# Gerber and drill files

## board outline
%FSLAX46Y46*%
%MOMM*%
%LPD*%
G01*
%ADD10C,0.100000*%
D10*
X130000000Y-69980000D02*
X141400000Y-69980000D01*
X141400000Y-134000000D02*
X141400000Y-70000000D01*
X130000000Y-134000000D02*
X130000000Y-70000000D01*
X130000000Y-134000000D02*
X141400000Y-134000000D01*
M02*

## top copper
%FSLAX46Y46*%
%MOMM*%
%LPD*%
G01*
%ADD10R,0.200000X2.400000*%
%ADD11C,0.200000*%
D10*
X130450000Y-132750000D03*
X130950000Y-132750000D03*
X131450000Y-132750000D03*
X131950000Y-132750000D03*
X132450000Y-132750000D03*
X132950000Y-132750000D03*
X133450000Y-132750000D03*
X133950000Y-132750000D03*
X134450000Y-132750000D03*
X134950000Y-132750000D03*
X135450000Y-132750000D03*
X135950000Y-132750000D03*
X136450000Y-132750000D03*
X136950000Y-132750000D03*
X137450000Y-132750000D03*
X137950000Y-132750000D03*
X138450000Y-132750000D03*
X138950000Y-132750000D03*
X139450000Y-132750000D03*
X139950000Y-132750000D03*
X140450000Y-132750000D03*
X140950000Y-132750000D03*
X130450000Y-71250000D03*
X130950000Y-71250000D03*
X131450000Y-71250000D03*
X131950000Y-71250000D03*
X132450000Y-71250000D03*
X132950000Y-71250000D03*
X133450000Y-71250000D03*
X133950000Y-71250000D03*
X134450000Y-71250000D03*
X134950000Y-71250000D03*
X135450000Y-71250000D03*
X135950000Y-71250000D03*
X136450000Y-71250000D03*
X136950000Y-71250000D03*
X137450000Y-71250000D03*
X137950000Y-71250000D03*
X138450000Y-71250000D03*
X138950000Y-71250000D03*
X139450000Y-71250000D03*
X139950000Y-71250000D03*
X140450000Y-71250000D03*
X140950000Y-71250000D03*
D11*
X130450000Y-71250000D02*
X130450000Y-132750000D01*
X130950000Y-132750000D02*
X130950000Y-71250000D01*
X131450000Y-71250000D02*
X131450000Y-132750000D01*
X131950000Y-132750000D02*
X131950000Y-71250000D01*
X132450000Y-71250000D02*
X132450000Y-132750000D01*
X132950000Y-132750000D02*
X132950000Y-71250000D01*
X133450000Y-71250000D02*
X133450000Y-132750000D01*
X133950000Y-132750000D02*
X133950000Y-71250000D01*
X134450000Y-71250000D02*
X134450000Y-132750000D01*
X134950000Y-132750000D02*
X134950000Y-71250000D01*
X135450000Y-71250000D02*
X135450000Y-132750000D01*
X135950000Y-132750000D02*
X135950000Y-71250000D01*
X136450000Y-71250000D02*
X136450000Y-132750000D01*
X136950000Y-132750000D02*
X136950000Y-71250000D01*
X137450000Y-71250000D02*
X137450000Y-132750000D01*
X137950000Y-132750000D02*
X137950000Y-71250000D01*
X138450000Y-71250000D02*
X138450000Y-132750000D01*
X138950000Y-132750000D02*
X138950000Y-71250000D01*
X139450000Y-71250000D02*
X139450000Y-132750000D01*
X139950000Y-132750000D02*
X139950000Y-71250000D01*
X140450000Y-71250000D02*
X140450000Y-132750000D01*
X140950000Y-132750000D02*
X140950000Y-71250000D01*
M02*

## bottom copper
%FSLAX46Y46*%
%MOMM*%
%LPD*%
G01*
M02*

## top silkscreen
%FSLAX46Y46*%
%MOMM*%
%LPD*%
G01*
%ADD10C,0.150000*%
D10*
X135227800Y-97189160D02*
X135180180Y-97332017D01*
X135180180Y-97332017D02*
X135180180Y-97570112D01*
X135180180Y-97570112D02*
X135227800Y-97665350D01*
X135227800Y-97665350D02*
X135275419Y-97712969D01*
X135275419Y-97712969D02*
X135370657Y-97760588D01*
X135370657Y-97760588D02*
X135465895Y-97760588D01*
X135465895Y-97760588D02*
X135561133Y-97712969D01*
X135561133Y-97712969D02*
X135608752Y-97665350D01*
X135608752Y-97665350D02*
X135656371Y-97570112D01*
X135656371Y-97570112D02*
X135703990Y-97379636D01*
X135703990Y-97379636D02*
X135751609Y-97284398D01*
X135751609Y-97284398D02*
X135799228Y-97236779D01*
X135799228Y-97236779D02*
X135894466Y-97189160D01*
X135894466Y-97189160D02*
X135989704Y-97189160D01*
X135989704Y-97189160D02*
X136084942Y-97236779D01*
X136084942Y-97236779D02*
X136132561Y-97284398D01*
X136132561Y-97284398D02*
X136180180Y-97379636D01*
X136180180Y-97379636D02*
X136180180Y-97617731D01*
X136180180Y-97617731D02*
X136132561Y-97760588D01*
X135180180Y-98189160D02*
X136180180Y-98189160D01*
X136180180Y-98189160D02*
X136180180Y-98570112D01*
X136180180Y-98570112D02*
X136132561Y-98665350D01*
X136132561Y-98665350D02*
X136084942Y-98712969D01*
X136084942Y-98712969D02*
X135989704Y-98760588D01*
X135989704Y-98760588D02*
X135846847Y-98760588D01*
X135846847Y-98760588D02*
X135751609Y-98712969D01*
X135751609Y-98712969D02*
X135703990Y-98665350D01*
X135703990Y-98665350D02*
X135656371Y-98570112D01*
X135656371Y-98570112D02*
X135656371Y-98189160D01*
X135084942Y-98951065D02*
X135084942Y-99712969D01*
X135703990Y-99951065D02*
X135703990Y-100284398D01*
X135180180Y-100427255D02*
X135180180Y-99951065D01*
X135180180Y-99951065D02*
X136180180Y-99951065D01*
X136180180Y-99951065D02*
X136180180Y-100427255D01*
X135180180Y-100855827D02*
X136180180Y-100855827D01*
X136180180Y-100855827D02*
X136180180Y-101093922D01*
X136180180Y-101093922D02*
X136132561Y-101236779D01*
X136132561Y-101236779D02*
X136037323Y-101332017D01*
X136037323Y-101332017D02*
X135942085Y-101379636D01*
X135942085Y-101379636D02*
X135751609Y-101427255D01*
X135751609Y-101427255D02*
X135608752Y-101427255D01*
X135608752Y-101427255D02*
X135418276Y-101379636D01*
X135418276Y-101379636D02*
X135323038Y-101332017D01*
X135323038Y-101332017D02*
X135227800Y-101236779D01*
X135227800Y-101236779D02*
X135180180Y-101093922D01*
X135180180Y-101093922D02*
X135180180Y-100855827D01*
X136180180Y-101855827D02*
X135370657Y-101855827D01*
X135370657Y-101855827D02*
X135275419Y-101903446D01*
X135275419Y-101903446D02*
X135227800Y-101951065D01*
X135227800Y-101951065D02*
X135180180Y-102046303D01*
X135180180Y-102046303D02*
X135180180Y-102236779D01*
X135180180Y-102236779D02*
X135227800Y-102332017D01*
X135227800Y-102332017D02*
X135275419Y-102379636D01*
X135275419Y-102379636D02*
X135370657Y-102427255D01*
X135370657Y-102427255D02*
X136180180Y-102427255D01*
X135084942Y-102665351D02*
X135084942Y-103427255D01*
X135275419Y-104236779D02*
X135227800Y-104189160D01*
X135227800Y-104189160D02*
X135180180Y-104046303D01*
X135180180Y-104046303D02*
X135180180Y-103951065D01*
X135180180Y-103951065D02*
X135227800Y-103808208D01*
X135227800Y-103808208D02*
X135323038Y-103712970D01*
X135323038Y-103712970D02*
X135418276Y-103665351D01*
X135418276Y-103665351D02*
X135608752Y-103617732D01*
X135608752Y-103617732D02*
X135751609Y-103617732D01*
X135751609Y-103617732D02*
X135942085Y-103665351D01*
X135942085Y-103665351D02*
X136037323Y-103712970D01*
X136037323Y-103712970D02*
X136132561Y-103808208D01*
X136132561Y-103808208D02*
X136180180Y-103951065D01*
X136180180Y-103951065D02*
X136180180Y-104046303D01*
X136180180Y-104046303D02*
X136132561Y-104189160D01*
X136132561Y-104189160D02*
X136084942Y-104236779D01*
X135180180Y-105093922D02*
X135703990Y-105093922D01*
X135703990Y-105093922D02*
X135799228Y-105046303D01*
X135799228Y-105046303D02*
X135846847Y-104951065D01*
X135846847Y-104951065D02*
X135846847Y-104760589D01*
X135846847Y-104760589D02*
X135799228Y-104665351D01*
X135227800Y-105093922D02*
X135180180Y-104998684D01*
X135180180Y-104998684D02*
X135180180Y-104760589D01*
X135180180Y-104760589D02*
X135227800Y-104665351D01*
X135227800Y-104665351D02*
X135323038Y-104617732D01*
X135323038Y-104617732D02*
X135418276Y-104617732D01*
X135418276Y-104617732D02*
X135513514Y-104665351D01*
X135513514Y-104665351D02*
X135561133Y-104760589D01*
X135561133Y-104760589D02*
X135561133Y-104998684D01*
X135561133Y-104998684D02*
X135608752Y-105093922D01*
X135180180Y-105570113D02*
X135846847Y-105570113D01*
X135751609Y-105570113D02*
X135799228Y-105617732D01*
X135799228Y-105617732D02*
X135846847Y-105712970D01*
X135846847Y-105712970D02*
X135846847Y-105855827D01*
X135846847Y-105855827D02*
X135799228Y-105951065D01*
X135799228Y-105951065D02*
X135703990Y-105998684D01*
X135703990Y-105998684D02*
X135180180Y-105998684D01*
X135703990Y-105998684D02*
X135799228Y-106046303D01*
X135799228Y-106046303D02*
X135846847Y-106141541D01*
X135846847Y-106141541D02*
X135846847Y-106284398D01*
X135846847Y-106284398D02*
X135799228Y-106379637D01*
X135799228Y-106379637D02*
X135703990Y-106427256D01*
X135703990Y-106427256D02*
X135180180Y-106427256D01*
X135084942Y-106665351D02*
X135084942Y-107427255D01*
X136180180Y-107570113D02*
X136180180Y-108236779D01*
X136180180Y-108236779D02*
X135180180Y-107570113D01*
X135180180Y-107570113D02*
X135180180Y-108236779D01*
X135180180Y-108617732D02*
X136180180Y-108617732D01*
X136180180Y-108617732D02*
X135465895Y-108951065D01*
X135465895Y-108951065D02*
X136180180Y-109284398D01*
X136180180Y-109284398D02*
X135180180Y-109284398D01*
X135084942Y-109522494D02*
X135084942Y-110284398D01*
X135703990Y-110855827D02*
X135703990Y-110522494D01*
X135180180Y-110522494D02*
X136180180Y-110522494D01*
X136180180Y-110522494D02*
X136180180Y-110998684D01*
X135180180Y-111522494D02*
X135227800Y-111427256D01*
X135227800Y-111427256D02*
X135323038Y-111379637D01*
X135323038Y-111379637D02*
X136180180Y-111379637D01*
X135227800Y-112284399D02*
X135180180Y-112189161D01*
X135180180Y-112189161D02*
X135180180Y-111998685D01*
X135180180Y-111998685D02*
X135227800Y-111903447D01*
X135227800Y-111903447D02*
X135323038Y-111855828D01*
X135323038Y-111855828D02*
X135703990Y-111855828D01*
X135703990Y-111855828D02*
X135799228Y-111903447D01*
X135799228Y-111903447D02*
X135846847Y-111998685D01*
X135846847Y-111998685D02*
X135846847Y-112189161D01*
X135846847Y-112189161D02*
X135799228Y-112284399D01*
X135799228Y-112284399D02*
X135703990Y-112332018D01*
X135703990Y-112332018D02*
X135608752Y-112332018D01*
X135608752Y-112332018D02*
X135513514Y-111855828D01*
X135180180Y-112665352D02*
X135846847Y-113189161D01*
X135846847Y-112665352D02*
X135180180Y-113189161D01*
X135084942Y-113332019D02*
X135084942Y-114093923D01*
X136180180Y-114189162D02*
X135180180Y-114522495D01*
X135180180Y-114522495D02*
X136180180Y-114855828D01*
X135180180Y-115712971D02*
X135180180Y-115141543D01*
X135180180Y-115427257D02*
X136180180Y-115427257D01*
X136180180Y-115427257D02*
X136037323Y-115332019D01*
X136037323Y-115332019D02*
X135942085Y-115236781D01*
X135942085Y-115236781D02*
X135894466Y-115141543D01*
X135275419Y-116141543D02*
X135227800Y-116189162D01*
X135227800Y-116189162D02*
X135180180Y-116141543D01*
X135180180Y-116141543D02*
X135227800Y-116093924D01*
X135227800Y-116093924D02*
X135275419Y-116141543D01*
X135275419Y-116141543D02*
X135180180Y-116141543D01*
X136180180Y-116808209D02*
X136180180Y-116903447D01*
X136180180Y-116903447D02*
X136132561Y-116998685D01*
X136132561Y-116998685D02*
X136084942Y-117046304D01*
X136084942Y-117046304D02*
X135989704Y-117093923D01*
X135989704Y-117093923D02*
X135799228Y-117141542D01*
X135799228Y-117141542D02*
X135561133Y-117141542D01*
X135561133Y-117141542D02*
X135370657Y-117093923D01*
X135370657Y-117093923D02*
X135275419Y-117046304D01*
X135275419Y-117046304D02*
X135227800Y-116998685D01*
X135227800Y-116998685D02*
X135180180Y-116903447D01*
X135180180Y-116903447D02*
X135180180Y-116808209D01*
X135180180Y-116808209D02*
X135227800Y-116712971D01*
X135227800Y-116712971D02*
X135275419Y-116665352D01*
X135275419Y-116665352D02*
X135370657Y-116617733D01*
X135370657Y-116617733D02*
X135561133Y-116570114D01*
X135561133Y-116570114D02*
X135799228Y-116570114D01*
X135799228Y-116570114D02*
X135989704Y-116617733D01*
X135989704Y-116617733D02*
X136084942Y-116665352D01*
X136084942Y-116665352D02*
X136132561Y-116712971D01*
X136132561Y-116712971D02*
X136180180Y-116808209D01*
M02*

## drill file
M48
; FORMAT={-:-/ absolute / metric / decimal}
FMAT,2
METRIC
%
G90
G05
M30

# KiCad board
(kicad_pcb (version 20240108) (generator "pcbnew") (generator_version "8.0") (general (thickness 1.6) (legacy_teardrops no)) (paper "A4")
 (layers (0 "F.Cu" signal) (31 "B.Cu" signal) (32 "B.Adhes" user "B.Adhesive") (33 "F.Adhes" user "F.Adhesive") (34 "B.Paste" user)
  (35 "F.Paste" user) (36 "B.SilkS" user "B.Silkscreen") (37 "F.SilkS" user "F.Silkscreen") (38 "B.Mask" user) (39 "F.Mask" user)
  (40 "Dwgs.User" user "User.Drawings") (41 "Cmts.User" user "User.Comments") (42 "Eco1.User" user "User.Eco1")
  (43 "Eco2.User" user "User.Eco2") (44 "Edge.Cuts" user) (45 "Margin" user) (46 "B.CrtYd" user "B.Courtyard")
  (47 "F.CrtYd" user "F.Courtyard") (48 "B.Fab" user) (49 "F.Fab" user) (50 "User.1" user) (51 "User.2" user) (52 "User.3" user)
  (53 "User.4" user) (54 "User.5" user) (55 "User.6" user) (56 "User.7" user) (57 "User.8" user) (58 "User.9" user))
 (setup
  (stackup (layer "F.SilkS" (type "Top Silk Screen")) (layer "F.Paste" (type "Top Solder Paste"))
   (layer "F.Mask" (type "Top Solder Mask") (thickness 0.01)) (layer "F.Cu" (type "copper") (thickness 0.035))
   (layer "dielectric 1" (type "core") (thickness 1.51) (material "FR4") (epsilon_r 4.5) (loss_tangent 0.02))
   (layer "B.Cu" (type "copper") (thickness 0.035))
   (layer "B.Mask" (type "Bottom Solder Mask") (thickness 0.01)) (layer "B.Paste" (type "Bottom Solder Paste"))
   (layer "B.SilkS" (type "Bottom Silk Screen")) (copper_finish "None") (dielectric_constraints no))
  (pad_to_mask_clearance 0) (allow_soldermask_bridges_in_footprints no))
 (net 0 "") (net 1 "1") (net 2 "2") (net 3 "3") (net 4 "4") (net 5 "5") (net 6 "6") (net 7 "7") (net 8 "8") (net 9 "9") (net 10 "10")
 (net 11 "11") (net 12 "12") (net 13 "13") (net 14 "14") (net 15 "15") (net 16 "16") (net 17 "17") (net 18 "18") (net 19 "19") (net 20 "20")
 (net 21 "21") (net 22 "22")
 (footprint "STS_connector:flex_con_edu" (layer "F.Cu") (at 130 136.1)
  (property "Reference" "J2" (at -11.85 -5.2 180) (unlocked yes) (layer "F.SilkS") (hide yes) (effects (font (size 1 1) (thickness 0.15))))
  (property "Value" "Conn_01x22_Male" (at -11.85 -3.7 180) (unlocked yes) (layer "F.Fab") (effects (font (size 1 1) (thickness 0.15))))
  (pad "1" smd rect (at 0.45 -3.35) (size 0.2 2.4) (layers "F.Cu" "F.Paste" "F.Mask") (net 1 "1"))
  (pad "2" smd rect (at 0.95 -3.35) (size 0.2 2.4) (layers "F.Cu" "F.Paste" "F.Mask") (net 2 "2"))
  (pad "3" smd rect (at 1.45 -3.35) (size 0.2 2.4) (layers "F.Cu" "F.Paste" "F.Mask") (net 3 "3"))
  (pad "4" smd rect (at 1.95 -3.35) (size 0.2 2.4) (layers "F.Cu" "F.Paste" "F.Mask") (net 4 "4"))
  (pad "5" smd rect (at 2.45 -3.35) (size 0.2 2.4) (layers "F.Cu" "F.Paste" "F.Mask") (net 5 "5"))
  (pad "6" smd rect (at 2.95 -3.35) (size 0.2 2.4) (layers "F.Cu" "F.Paste" "F.Mask") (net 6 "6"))
  (pad "7" smd rect (at 3.45 -3.35) (size 0.2 2.4) (layers "F.Cu" "F.Paste" "F.Mask") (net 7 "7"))
  (pad "8" smd rect (at 3.95 -3.35) (size 0.2 2.4) (layers "F.Cu" "F.Paste" "F.Mask") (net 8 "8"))
  (pad "9" smd rect (at 4.45 -3.35) (size 0.2 2.4) (layers "F.Cu" "F.Paste" "F.Mask") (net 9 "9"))
  (pad "10" smd rect (at 4.95 -3.35) (size 0.2 2.4) (layers "F.Cu" "F.Paste" "F.Mask") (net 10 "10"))
  (pad "11" smd rect (at 5.45 -3.35) (size 0.2 2.4) (layers "F.Cu" "F.Paste" "F.Mask") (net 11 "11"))
  (pad "12" smd rect (at 5.95 -3.35) (size 0.2 2.4) (layers "F.Cu" "F.Paste" "F.Mask") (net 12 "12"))
  (pad "13" smd rect (at 6.45 -3.35) (size 0.2 2.4) (layers "F.Cu" "F.Paste" "F.Mask") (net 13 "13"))
  (pad "14" smd rect (at 6.95 -3.35) (size 0.2 2.4) (layers "F.Cu" "F.Paste" "F.Mask") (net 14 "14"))
  (pad "15" smd rect (at 7.45 -3.35) (size 0.2 2.4) (layers "F.Cu" "F.Paste" "F.Mask") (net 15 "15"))
  (pad "16" smd rect (at 7.95 -3.35) (size 0.2 2.4) (layers "F.Cu" "F.Paste" "F.Mask") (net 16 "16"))
  (pad "17" smd rect (at 8.45 -3.35) (size 0.2 2.4) (layers "F.Cu" "F.Paste" "F.Mask") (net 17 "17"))
  (pad "18" smd rect (at 8.95 -3.35) (size 0.2 2.4) (layers "F.Cu" "F.Paste" "F.Mask") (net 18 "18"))
  (pad "19" smd rect (at 9.45 -3.35) (size 0.2 2.4) (layers "F.Cu" "F.Paste" "F.Mask") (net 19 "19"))
  (pad "20" smd rect (at 9.95 -3.35) (size 0.2 2.4) (layers "F.Cu" "F.Paste" "F.Mask") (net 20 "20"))
  (pad "21" smd rect (at 10.45 -3.35) (size 0.2 2.4) (layers "F.Cu" "F.Paste" "F.Mask") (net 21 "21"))
  (pad "22" smd rect (at 10.95 -3.35) (size 0.2 2.4) (layers "F.Cu" "F.Paste" "F.Mask") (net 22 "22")))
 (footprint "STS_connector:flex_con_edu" (layer "F.Cu") (at 130 74.6)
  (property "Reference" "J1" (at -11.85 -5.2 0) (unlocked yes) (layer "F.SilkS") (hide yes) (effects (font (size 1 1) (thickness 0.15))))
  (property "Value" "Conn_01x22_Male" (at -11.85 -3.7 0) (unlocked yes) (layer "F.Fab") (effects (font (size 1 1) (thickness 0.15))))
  (pad "1" smd rect (at 0.45 -3.35) (size 0.2 2.4) (layers "F.Cu" "F.Paste" "F.Mask") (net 1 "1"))
  (pad "2" smd rect (at 0.95 -3.35) (size 0.2 2.4) (layers "F.Cu" "F.Paste" "F.Mask") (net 2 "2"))
  (pad "3" smd rect (at 1.45 -3.35) (size 0.2 2.4) (layers "F.Cu" "F.Paste" "F.Mask") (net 3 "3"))
  (pad "4" smd rect (at 1.95 -3.35) (size 0.2 2.4) (layers "F.Cu" "F.Paste" "F.Mask") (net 4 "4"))
  (pad "5" smd rect (at 2.45 -3.35) (size 0.2 2.4) (layers "F.Cu" "F.Paste" "F.Mask") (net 5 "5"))
  (pad "6" smd rect (at 2.95 -3.35) (size 0.2 2.4) (layers "F.Cu" "F.Paste" "F.Mask") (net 6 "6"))
  (pad "7" smd rect (at 3.45 -3.35) (size 0.2 2.4) (layers "F.Cu" "F.Paste" "F.Mask") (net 7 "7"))
  (pad "8" smd rect (at 3.95 -3.35) (size 0.2 2.4) (layers "F.Cu" "F.Paste" "F.Mask") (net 8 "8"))
  (pad "9" smd rect (at 4.45 -3.35) (size 0.2 2.4) (layers "F.Cu" "F.Paste" "F.Mask") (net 9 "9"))
  (pad "10" smd rect (at 4.95 -3.35) (size 0.2 2.4) (layers "F.Cu" "F.Paste" "F.Mask") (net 10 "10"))
  (pad "11" smd rect (at 5.45 -3.35) (size 0.2 2.4) (layers "F.Cu" "F.Paste" "F.Mask") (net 11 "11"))
  (pad "12" smd rect (at 5.95 -3.35) (size 0.2 2.4) (layers "F.Cu" "F.Paste" "F.Mask") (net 12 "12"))
  (pad "13" smd rect (at 6.45 -3.35) (size 0.2 2.4) (layers "F.Cu" "F.Paste" "F.Mask") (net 13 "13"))
  (pad "14" smd rect (at 6.95 -3.35) (size 0.2 2.4) (layers "F.Cu" "F.Paste" "F.Mask") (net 14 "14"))
  (pad "15" smd rect (at 7.45 -3.35) (size 0.2 2.4) (layers "F.Cu" "F.Paste" "F.Mask") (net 15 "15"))
  (pad "16" smd rect (at 7.95 -3.35) (size 0.2 2.4) (layers "F.Cu" "F.Paste" "F.Mask") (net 16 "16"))
  (pad "17" smd rect (at 8.45 -3.35) (size 0.2 2.4) (layers "F.Cu" "F.Paste" "F.Mask") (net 17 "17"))
  (pad "18" smd rect (at 8.95 -3.35) (size 0.2 2.4) (layers "F.Cu" "F.Paste" "F.Mask") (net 18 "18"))
  (pad "19" smd rect (at 9.45 -3.35) (size 0.2 2.4) (layers "F.Cu" "F.Paste" "F.Mask") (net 19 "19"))
  (pad "20" smd rect (at 9.95 -3.35) (size 0.2 2.4) (layers "F.Cu" "F.Paste" "F.Mask") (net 20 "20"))
  (pad "21" smd rect (at 10.45 -3.35) (size 0.2 2.4) (layers "F.Cu" "F.Paste" "F.Mask") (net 21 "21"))
  (pad "22" smd rect (at 10.95 -3.35) (size 0.2 2.4) (layers "F.Cu" "F.Paste" "F.Mask") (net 22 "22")))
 (gr_line (start 130 69.98) (end 141.4 69.98) (stroke (width 0.1) (type solid)) (layer "Edge.Cuts"))
 (gr_line (start 141.4 134) (end 141.4 70) (stroke (width 0.1) (type solid)) (layer "Edge.Cuts"))
 (gr_line (start 130 134) (end 130 70) (stroke (width 0.1) (type solid)) (layer "Edge.Cuts"))
 (gr_line (start 130 134) (end 141.4 134) (stroke (width 0.1) (type solid)) (layer "Edge.Cuts"))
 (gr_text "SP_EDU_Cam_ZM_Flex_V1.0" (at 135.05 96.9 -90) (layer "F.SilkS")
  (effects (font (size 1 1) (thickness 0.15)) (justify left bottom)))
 (segment (start 130.45 71.25) (end 130.45 132.75) (width 0.2) (layer "F.Cu") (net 1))
 (segment (start 130.95 132.75) (end 130.95 71.25) (width 0.2) (layer "F.Cu") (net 2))
 (segment (start 131.45 71.25) (end 131.45 132.75) (width 0.2) (layer "F.Cu") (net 3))
 (segment (start 131.95 132.75) (end 131.95 71.25) (width 0.2) (layer "F.Cu") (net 4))
 (segment (start 132.45 71.25) (end 132.45 132.75) (width 0.2) (layer "F.Cu") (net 5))
 (segment (start 132.95 132.75) (end 132.95 71.25) (width 0.2) (layer "F.Cu") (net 6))
 (segment (start 133.45 71.25) (end 133.45 132.75) (width 0.2) (layer "F.Cu") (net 7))
 (segment (start 133.95 132.75) (end 133.95 71.25) (width 0.2) (layer "F.Cu") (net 8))
 (segment (start 134.45 71.25) (end 134.45 132.75) (width 0.2) (layer "F.Cu") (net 9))
 (segment (start 134.95 132.75) (end 134.95 71.25) (width 0.2) (layer "F.Cu") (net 10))
 (segment (start 135.45 71.25) (end 135.45 132.75) (width 0.2) (layer "F.Cu") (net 11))
 (segment (start 135.95 132.75) (end 135.95 71.25) (width 0.2) (layer "F.Cu") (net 12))
 (segment (start 136.45 71.25) (end 136.45 132.75) (width 0.2) (layer "F.Cu") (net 13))
 (segment (start 136.95 132.75) (end 136.95 71.25) (width 0.2) (layer "F.Cu") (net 14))
 (segment (start 137.45 71.25) (end 137.45 132.75) (width 0.2) (layer "F.Cu") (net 15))
 (segment (start 137.95 132.75) (end 137.95 71.25) (width 0.2) (layer "F.Cu") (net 16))
 (segment (start 138.45 71.25) (end 138.45 132.75) (width 0.2) (layer "F.Cu") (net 17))
 (segment (start 138.95 132.75) (end 138.95 71.25) (width 0.2) (layer "F.Cu") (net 18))
 (segment (start 139.45 71.25) (end 139.45 132.75) (width 0.2) (layer "F.Cu") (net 19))
 (segment (start 139.95 132.75) (end 139.95 71.25) (width 0.2) (layer "F.Cu") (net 20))
 (segment (start 140.45 71.25) (end 140.45 132.75) (width 0.2) (layer "F.Cu") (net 21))
 (segment (start 140.95 132.75) (end 140.95 71.25) (width 0.2) (layer "F.Cu") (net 22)))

